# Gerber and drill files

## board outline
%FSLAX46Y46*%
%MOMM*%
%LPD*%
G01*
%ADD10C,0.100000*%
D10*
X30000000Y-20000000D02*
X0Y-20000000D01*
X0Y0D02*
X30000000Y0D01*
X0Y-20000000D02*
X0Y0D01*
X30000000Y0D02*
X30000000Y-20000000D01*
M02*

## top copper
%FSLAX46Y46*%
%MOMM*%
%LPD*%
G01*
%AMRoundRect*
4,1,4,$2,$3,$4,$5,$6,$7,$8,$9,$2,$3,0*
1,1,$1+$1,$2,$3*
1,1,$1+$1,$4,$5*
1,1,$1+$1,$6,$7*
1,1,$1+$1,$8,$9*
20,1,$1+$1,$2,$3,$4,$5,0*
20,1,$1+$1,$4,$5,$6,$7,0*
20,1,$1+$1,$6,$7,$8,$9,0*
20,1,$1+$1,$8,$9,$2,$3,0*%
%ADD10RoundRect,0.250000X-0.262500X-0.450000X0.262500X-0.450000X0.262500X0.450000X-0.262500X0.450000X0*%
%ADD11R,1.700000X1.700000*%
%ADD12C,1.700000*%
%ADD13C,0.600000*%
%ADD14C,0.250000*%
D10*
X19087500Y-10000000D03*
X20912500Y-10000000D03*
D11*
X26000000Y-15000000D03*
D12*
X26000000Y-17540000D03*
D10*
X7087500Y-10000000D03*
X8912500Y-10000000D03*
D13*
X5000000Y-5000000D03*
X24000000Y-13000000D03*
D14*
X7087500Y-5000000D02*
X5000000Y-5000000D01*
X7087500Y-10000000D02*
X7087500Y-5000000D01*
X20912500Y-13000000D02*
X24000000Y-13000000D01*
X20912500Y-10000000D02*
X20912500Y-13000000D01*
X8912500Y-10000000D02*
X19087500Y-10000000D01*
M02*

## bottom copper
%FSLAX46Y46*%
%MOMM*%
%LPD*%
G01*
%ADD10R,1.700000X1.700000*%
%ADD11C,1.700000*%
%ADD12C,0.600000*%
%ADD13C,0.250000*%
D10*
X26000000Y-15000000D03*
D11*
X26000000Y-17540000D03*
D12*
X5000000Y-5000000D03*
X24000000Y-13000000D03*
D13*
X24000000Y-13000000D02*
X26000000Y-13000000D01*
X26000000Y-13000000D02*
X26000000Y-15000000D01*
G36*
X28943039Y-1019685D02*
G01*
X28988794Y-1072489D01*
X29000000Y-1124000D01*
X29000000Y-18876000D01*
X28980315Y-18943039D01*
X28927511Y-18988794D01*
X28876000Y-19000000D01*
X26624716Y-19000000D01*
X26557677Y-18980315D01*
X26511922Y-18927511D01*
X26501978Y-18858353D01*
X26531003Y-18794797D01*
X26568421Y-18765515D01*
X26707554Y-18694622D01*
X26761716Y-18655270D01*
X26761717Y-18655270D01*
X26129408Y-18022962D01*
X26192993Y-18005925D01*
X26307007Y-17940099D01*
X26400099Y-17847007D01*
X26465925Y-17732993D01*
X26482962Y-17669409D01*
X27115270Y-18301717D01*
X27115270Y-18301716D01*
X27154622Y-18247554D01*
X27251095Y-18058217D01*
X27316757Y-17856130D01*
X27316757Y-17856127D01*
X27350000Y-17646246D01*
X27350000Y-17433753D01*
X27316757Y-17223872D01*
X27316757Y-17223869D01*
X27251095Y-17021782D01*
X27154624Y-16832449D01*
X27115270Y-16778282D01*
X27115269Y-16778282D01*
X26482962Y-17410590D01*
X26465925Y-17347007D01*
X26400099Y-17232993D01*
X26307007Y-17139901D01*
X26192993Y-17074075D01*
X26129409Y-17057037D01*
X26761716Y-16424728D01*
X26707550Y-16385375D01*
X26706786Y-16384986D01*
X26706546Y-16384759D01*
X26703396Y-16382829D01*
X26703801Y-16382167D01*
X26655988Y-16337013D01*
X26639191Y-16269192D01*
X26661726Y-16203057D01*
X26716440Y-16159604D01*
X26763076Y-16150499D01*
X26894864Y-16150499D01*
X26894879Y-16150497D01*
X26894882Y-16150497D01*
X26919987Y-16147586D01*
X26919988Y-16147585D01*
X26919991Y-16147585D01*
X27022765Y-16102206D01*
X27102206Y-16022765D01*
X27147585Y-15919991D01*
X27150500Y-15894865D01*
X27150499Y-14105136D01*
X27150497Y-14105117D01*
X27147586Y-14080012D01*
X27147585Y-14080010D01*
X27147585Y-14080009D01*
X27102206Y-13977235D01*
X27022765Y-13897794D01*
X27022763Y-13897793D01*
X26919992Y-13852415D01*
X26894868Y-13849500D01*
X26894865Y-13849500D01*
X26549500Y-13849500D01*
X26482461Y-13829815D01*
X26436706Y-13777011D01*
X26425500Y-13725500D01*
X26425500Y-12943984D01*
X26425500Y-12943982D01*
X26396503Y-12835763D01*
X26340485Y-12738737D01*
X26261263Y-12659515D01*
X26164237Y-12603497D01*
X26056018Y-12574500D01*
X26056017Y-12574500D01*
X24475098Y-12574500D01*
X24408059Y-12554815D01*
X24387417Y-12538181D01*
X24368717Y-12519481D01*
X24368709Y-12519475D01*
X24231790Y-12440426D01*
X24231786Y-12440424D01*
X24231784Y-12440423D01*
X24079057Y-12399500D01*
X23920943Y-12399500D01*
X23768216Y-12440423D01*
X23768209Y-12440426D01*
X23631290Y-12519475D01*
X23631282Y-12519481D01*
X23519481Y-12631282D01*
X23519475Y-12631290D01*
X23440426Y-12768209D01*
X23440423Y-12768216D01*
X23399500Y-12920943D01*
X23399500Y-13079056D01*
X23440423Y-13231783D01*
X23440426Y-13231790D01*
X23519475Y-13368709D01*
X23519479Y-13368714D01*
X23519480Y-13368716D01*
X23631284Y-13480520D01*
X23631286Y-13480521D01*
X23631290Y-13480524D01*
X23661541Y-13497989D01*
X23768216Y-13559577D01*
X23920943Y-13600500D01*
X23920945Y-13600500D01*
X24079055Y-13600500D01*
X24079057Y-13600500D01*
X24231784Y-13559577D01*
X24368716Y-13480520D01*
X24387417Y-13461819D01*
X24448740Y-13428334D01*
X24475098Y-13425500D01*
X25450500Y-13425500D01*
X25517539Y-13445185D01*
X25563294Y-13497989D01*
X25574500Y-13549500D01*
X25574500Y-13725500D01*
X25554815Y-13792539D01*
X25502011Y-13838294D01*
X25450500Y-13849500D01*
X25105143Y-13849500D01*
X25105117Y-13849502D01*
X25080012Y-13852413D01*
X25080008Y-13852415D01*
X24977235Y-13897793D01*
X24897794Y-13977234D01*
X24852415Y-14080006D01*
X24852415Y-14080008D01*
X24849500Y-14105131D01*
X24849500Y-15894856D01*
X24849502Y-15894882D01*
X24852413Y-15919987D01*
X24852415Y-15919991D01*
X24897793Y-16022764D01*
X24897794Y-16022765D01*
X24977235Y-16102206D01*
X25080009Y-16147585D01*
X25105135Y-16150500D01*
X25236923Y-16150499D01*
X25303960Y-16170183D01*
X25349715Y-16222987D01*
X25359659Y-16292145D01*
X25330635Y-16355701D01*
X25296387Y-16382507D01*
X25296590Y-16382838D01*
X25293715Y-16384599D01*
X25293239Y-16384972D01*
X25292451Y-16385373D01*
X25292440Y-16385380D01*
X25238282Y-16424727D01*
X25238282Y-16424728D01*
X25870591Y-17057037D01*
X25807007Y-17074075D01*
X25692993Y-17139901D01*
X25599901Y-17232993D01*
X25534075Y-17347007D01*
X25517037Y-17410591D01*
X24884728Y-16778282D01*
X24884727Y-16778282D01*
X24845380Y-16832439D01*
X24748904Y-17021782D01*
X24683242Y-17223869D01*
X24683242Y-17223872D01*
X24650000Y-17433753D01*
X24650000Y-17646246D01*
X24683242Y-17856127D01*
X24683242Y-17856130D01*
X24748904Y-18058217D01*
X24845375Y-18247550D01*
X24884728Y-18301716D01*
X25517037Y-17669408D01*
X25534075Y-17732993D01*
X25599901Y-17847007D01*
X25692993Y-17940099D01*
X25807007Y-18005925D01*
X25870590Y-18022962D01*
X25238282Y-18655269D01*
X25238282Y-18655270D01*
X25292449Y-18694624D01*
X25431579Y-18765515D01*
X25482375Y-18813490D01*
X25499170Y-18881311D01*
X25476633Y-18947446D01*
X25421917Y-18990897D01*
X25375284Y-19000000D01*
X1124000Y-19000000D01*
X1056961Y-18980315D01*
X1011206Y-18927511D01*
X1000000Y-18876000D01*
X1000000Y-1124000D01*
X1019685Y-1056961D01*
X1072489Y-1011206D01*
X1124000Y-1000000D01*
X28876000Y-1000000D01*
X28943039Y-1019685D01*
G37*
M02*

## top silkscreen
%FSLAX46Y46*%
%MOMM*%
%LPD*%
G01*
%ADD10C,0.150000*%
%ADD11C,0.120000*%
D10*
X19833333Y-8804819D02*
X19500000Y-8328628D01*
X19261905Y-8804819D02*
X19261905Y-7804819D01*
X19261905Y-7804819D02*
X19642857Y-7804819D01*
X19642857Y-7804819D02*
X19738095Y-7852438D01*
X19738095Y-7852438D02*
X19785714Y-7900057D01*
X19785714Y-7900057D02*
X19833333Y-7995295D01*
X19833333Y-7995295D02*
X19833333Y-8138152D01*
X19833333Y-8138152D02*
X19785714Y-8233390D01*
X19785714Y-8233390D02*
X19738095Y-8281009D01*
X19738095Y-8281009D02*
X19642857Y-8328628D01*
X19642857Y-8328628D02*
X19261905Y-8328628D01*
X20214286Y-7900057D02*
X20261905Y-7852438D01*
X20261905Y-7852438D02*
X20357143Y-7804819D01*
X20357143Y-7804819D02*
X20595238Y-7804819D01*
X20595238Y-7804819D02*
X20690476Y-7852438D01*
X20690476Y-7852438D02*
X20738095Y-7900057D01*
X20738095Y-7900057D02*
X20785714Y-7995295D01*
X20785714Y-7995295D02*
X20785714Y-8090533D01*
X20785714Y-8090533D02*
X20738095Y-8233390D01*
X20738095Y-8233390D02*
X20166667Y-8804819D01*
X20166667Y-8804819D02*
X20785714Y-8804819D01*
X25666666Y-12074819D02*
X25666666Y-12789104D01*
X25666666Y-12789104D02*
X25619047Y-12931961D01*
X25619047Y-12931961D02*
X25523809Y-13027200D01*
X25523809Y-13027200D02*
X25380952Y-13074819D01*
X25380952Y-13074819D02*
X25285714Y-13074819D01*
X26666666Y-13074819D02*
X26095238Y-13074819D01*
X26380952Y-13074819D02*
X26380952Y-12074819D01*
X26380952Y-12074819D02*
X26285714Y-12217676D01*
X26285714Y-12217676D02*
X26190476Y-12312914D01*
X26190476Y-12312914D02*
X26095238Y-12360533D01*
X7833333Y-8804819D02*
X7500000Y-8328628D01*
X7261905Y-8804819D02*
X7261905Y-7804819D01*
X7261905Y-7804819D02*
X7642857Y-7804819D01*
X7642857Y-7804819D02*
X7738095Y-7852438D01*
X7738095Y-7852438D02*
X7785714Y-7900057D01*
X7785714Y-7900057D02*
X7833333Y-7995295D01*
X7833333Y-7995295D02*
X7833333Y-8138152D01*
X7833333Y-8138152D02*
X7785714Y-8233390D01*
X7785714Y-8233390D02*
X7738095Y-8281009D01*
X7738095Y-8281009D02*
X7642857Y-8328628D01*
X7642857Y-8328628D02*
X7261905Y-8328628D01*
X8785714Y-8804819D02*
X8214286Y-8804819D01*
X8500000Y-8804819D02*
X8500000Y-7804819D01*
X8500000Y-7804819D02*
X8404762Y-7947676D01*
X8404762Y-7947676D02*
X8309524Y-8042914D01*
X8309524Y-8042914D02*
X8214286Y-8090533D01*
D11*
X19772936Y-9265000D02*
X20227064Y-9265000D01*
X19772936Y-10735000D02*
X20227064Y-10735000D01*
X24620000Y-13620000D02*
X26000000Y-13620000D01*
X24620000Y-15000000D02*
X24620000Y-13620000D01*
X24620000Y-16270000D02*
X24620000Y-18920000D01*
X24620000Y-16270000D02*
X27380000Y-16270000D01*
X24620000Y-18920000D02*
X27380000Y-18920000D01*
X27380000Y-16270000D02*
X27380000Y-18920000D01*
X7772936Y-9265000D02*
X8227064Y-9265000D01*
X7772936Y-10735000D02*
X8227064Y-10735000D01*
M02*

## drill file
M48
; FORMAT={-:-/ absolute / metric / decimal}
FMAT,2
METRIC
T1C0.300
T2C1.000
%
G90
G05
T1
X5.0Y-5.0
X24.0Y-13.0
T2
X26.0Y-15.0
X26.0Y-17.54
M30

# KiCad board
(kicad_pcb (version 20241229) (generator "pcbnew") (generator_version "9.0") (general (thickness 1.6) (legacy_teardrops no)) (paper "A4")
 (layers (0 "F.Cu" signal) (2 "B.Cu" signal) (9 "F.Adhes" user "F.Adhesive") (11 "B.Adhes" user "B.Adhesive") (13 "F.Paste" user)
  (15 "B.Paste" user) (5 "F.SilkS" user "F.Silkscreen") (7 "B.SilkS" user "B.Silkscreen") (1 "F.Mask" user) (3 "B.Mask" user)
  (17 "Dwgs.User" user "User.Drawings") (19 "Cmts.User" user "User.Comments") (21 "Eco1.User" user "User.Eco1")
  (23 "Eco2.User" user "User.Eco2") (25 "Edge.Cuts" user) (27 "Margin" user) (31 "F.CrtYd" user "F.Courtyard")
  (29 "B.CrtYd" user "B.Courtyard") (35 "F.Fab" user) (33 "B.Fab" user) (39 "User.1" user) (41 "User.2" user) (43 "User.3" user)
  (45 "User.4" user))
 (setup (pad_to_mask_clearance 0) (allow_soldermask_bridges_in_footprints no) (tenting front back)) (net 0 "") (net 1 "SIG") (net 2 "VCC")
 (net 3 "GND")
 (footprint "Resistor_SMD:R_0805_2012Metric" (layer "F.Cu") (at 20 10)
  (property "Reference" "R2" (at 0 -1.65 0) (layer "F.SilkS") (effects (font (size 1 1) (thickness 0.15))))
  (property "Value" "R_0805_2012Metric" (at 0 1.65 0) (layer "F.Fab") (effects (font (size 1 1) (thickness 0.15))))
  (fp_line (start -0.227064 -0.735) (end 0.227064 -0.735) (stroke (width 0.12) (type solid)) (layer "F.SilkS"))
  (fp_line (start -0.227064 0.735) (end 0.227064 0.735) (stroke (width 0.12) (type solid)) (layer "F.SilkS"))
  (pad "1" smd roundrect (at -0.9125 0) (size 1.025 1.4) (layers "F.Cu" "F.Mask" "F.Paste") (roundrect_rratio 0.243902) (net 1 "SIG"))
  (pad "2" smd roundrect (at 0.9125 0) (size 1.025 1.4) (layers "F.Cu" "F.Mask" "F.Paste") (roundrect_rratio 0.243902) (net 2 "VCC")))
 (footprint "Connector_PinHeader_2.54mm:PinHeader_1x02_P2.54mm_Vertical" (layer "F.Cu") (at 26 15)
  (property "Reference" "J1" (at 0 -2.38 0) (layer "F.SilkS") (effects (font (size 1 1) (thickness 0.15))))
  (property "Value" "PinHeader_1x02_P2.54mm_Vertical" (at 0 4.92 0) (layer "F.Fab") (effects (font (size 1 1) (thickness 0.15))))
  (fp_line (start -1.38 -1.38) (end 0 -1.38) (stroke (width 0.12) (type solid)) (layer "F.SilkS"))
  (fp_line (start -1.38 0) (end -1.38 -1.38) (stroke (width 0.12) (type solid)) (layer "F.SilkS"))
  (fp_line (start -1.38 1.27) (end -1.38 3.92) (stroke (width 0.12) (type solid)) (layer "F.SilkS"))
  (fp_line (start -1.38 1.27) (end 1.38 1.27) (stroke (width 0.12) (type solid)) (layer "F.SilkS"))
  (fp_line (start -1.38 3.92) (end 1.38 3.92) (stroke (width 0.12) (type solid)) (layer "F.SilkS"))
  (fp_line (start 1.38 1.27) (end 1.38 3.92) (stroke (width 0.12) (type solid)) (layer "F.SilkS"))
  (pad "1" thru_hole rect (at 0 0) (size 1.7 1.7) (drill 1) (layers "*.Cu" "*.Mask") (remove_unused_layers no) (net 2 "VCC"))
  (pad "2" thru_hole circle (at 0 2.54) (size 1.7 1.7) (drill 1) (layers "*.Cu" "*.Mask") (remove_unused_layers no) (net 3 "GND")))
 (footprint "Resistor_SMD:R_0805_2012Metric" (layer "F.Cu") (at 8 10)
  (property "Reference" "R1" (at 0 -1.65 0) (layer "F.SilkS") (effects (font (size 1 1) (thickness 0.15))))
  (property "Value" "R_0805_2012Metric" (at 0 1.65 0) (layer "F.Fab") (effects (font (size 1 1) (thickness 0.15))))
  (fp_line (start -0.227064 -0.735) (end 0.227064 -0.735) (stroke (width 0.12) (type solid)) (layer "F.SilkS"))
  (fp_line (start -0.227064 0.735) (end 0.227064 0.735) (stroke (width 0.12) (type solid)) (layer "F.SilkS"))
  (pad "1" smd roundrect (at -0.9125 0) (size 1.025 1.4) (layers "F.Cu" "F.Mask" "F.Paste") (roundrect_rratio 0.243902) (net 3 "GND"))
  (pad "2" smd roundrect (at 0.9125 0) (size 1.025 1.4) (layers "F.Cu" "F.Mask" "F.Paste") (roundrect_rratio 0.243902) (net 1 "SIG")))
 (gr_line (start 30 20) (end 0 20) (stroke (width 0.1) (type default)) (layer "Edge.Cuts"))
 (gr_line (start 0 0) (end 30 0) (stroke (width 0.1) (type default)) (layer "Edge.Cuts"))
 (gr_line (start 0 20) (end 0 0) (stroke (width 0.1) (type default)) (layer "Edge.Cuts"))
 (gr_line (start 30 0) (end 30 20) (stroke (width 0.1) (type default)) (layer "Edge.Cuts"))
 (segment (start 7.0875 5) (end 5 5) (width 0.25) (layer "F.Cu") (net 3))
 (segment (start 7.0875 10) (end 7.0875 5) (width 0.25) (layer "F.Cu") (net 3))
 (via (at 5 5) (size 0.6) (drill 0.3) (layers "F.Cu" "B.Cu") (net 3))
 (segment (start 20.9125 13) (end 24 13) (width 0.25) (layer "F.Cu") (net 2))
 (segment (start 20.9125 10) (end 20.9125 13) (width 0.25) (layer "F.Cu") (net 2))
 (via (at 24 13) (size 0.6) (drill 0.3) (layers "F.Cu" "B.Cu") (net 2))
 (segment (start 24 13) (end 26 13) (width 0.25) (layer "B.Cu") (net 2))
 (segment (start 26 13) (end 26 15) (width 0.25) (layer "B.Cu") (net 2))
 (segment (start 8.9125 10) (end 19.0875 10) (width 0.25) (layer "F.Cu") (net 1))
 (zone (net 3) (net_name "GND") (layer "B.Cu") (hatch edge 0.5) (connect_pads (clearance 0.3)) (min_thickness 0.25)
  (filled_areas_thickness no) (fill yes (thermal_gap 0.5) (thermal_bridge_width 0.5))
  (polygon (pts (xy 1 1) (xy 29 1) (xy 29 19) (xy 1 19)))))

